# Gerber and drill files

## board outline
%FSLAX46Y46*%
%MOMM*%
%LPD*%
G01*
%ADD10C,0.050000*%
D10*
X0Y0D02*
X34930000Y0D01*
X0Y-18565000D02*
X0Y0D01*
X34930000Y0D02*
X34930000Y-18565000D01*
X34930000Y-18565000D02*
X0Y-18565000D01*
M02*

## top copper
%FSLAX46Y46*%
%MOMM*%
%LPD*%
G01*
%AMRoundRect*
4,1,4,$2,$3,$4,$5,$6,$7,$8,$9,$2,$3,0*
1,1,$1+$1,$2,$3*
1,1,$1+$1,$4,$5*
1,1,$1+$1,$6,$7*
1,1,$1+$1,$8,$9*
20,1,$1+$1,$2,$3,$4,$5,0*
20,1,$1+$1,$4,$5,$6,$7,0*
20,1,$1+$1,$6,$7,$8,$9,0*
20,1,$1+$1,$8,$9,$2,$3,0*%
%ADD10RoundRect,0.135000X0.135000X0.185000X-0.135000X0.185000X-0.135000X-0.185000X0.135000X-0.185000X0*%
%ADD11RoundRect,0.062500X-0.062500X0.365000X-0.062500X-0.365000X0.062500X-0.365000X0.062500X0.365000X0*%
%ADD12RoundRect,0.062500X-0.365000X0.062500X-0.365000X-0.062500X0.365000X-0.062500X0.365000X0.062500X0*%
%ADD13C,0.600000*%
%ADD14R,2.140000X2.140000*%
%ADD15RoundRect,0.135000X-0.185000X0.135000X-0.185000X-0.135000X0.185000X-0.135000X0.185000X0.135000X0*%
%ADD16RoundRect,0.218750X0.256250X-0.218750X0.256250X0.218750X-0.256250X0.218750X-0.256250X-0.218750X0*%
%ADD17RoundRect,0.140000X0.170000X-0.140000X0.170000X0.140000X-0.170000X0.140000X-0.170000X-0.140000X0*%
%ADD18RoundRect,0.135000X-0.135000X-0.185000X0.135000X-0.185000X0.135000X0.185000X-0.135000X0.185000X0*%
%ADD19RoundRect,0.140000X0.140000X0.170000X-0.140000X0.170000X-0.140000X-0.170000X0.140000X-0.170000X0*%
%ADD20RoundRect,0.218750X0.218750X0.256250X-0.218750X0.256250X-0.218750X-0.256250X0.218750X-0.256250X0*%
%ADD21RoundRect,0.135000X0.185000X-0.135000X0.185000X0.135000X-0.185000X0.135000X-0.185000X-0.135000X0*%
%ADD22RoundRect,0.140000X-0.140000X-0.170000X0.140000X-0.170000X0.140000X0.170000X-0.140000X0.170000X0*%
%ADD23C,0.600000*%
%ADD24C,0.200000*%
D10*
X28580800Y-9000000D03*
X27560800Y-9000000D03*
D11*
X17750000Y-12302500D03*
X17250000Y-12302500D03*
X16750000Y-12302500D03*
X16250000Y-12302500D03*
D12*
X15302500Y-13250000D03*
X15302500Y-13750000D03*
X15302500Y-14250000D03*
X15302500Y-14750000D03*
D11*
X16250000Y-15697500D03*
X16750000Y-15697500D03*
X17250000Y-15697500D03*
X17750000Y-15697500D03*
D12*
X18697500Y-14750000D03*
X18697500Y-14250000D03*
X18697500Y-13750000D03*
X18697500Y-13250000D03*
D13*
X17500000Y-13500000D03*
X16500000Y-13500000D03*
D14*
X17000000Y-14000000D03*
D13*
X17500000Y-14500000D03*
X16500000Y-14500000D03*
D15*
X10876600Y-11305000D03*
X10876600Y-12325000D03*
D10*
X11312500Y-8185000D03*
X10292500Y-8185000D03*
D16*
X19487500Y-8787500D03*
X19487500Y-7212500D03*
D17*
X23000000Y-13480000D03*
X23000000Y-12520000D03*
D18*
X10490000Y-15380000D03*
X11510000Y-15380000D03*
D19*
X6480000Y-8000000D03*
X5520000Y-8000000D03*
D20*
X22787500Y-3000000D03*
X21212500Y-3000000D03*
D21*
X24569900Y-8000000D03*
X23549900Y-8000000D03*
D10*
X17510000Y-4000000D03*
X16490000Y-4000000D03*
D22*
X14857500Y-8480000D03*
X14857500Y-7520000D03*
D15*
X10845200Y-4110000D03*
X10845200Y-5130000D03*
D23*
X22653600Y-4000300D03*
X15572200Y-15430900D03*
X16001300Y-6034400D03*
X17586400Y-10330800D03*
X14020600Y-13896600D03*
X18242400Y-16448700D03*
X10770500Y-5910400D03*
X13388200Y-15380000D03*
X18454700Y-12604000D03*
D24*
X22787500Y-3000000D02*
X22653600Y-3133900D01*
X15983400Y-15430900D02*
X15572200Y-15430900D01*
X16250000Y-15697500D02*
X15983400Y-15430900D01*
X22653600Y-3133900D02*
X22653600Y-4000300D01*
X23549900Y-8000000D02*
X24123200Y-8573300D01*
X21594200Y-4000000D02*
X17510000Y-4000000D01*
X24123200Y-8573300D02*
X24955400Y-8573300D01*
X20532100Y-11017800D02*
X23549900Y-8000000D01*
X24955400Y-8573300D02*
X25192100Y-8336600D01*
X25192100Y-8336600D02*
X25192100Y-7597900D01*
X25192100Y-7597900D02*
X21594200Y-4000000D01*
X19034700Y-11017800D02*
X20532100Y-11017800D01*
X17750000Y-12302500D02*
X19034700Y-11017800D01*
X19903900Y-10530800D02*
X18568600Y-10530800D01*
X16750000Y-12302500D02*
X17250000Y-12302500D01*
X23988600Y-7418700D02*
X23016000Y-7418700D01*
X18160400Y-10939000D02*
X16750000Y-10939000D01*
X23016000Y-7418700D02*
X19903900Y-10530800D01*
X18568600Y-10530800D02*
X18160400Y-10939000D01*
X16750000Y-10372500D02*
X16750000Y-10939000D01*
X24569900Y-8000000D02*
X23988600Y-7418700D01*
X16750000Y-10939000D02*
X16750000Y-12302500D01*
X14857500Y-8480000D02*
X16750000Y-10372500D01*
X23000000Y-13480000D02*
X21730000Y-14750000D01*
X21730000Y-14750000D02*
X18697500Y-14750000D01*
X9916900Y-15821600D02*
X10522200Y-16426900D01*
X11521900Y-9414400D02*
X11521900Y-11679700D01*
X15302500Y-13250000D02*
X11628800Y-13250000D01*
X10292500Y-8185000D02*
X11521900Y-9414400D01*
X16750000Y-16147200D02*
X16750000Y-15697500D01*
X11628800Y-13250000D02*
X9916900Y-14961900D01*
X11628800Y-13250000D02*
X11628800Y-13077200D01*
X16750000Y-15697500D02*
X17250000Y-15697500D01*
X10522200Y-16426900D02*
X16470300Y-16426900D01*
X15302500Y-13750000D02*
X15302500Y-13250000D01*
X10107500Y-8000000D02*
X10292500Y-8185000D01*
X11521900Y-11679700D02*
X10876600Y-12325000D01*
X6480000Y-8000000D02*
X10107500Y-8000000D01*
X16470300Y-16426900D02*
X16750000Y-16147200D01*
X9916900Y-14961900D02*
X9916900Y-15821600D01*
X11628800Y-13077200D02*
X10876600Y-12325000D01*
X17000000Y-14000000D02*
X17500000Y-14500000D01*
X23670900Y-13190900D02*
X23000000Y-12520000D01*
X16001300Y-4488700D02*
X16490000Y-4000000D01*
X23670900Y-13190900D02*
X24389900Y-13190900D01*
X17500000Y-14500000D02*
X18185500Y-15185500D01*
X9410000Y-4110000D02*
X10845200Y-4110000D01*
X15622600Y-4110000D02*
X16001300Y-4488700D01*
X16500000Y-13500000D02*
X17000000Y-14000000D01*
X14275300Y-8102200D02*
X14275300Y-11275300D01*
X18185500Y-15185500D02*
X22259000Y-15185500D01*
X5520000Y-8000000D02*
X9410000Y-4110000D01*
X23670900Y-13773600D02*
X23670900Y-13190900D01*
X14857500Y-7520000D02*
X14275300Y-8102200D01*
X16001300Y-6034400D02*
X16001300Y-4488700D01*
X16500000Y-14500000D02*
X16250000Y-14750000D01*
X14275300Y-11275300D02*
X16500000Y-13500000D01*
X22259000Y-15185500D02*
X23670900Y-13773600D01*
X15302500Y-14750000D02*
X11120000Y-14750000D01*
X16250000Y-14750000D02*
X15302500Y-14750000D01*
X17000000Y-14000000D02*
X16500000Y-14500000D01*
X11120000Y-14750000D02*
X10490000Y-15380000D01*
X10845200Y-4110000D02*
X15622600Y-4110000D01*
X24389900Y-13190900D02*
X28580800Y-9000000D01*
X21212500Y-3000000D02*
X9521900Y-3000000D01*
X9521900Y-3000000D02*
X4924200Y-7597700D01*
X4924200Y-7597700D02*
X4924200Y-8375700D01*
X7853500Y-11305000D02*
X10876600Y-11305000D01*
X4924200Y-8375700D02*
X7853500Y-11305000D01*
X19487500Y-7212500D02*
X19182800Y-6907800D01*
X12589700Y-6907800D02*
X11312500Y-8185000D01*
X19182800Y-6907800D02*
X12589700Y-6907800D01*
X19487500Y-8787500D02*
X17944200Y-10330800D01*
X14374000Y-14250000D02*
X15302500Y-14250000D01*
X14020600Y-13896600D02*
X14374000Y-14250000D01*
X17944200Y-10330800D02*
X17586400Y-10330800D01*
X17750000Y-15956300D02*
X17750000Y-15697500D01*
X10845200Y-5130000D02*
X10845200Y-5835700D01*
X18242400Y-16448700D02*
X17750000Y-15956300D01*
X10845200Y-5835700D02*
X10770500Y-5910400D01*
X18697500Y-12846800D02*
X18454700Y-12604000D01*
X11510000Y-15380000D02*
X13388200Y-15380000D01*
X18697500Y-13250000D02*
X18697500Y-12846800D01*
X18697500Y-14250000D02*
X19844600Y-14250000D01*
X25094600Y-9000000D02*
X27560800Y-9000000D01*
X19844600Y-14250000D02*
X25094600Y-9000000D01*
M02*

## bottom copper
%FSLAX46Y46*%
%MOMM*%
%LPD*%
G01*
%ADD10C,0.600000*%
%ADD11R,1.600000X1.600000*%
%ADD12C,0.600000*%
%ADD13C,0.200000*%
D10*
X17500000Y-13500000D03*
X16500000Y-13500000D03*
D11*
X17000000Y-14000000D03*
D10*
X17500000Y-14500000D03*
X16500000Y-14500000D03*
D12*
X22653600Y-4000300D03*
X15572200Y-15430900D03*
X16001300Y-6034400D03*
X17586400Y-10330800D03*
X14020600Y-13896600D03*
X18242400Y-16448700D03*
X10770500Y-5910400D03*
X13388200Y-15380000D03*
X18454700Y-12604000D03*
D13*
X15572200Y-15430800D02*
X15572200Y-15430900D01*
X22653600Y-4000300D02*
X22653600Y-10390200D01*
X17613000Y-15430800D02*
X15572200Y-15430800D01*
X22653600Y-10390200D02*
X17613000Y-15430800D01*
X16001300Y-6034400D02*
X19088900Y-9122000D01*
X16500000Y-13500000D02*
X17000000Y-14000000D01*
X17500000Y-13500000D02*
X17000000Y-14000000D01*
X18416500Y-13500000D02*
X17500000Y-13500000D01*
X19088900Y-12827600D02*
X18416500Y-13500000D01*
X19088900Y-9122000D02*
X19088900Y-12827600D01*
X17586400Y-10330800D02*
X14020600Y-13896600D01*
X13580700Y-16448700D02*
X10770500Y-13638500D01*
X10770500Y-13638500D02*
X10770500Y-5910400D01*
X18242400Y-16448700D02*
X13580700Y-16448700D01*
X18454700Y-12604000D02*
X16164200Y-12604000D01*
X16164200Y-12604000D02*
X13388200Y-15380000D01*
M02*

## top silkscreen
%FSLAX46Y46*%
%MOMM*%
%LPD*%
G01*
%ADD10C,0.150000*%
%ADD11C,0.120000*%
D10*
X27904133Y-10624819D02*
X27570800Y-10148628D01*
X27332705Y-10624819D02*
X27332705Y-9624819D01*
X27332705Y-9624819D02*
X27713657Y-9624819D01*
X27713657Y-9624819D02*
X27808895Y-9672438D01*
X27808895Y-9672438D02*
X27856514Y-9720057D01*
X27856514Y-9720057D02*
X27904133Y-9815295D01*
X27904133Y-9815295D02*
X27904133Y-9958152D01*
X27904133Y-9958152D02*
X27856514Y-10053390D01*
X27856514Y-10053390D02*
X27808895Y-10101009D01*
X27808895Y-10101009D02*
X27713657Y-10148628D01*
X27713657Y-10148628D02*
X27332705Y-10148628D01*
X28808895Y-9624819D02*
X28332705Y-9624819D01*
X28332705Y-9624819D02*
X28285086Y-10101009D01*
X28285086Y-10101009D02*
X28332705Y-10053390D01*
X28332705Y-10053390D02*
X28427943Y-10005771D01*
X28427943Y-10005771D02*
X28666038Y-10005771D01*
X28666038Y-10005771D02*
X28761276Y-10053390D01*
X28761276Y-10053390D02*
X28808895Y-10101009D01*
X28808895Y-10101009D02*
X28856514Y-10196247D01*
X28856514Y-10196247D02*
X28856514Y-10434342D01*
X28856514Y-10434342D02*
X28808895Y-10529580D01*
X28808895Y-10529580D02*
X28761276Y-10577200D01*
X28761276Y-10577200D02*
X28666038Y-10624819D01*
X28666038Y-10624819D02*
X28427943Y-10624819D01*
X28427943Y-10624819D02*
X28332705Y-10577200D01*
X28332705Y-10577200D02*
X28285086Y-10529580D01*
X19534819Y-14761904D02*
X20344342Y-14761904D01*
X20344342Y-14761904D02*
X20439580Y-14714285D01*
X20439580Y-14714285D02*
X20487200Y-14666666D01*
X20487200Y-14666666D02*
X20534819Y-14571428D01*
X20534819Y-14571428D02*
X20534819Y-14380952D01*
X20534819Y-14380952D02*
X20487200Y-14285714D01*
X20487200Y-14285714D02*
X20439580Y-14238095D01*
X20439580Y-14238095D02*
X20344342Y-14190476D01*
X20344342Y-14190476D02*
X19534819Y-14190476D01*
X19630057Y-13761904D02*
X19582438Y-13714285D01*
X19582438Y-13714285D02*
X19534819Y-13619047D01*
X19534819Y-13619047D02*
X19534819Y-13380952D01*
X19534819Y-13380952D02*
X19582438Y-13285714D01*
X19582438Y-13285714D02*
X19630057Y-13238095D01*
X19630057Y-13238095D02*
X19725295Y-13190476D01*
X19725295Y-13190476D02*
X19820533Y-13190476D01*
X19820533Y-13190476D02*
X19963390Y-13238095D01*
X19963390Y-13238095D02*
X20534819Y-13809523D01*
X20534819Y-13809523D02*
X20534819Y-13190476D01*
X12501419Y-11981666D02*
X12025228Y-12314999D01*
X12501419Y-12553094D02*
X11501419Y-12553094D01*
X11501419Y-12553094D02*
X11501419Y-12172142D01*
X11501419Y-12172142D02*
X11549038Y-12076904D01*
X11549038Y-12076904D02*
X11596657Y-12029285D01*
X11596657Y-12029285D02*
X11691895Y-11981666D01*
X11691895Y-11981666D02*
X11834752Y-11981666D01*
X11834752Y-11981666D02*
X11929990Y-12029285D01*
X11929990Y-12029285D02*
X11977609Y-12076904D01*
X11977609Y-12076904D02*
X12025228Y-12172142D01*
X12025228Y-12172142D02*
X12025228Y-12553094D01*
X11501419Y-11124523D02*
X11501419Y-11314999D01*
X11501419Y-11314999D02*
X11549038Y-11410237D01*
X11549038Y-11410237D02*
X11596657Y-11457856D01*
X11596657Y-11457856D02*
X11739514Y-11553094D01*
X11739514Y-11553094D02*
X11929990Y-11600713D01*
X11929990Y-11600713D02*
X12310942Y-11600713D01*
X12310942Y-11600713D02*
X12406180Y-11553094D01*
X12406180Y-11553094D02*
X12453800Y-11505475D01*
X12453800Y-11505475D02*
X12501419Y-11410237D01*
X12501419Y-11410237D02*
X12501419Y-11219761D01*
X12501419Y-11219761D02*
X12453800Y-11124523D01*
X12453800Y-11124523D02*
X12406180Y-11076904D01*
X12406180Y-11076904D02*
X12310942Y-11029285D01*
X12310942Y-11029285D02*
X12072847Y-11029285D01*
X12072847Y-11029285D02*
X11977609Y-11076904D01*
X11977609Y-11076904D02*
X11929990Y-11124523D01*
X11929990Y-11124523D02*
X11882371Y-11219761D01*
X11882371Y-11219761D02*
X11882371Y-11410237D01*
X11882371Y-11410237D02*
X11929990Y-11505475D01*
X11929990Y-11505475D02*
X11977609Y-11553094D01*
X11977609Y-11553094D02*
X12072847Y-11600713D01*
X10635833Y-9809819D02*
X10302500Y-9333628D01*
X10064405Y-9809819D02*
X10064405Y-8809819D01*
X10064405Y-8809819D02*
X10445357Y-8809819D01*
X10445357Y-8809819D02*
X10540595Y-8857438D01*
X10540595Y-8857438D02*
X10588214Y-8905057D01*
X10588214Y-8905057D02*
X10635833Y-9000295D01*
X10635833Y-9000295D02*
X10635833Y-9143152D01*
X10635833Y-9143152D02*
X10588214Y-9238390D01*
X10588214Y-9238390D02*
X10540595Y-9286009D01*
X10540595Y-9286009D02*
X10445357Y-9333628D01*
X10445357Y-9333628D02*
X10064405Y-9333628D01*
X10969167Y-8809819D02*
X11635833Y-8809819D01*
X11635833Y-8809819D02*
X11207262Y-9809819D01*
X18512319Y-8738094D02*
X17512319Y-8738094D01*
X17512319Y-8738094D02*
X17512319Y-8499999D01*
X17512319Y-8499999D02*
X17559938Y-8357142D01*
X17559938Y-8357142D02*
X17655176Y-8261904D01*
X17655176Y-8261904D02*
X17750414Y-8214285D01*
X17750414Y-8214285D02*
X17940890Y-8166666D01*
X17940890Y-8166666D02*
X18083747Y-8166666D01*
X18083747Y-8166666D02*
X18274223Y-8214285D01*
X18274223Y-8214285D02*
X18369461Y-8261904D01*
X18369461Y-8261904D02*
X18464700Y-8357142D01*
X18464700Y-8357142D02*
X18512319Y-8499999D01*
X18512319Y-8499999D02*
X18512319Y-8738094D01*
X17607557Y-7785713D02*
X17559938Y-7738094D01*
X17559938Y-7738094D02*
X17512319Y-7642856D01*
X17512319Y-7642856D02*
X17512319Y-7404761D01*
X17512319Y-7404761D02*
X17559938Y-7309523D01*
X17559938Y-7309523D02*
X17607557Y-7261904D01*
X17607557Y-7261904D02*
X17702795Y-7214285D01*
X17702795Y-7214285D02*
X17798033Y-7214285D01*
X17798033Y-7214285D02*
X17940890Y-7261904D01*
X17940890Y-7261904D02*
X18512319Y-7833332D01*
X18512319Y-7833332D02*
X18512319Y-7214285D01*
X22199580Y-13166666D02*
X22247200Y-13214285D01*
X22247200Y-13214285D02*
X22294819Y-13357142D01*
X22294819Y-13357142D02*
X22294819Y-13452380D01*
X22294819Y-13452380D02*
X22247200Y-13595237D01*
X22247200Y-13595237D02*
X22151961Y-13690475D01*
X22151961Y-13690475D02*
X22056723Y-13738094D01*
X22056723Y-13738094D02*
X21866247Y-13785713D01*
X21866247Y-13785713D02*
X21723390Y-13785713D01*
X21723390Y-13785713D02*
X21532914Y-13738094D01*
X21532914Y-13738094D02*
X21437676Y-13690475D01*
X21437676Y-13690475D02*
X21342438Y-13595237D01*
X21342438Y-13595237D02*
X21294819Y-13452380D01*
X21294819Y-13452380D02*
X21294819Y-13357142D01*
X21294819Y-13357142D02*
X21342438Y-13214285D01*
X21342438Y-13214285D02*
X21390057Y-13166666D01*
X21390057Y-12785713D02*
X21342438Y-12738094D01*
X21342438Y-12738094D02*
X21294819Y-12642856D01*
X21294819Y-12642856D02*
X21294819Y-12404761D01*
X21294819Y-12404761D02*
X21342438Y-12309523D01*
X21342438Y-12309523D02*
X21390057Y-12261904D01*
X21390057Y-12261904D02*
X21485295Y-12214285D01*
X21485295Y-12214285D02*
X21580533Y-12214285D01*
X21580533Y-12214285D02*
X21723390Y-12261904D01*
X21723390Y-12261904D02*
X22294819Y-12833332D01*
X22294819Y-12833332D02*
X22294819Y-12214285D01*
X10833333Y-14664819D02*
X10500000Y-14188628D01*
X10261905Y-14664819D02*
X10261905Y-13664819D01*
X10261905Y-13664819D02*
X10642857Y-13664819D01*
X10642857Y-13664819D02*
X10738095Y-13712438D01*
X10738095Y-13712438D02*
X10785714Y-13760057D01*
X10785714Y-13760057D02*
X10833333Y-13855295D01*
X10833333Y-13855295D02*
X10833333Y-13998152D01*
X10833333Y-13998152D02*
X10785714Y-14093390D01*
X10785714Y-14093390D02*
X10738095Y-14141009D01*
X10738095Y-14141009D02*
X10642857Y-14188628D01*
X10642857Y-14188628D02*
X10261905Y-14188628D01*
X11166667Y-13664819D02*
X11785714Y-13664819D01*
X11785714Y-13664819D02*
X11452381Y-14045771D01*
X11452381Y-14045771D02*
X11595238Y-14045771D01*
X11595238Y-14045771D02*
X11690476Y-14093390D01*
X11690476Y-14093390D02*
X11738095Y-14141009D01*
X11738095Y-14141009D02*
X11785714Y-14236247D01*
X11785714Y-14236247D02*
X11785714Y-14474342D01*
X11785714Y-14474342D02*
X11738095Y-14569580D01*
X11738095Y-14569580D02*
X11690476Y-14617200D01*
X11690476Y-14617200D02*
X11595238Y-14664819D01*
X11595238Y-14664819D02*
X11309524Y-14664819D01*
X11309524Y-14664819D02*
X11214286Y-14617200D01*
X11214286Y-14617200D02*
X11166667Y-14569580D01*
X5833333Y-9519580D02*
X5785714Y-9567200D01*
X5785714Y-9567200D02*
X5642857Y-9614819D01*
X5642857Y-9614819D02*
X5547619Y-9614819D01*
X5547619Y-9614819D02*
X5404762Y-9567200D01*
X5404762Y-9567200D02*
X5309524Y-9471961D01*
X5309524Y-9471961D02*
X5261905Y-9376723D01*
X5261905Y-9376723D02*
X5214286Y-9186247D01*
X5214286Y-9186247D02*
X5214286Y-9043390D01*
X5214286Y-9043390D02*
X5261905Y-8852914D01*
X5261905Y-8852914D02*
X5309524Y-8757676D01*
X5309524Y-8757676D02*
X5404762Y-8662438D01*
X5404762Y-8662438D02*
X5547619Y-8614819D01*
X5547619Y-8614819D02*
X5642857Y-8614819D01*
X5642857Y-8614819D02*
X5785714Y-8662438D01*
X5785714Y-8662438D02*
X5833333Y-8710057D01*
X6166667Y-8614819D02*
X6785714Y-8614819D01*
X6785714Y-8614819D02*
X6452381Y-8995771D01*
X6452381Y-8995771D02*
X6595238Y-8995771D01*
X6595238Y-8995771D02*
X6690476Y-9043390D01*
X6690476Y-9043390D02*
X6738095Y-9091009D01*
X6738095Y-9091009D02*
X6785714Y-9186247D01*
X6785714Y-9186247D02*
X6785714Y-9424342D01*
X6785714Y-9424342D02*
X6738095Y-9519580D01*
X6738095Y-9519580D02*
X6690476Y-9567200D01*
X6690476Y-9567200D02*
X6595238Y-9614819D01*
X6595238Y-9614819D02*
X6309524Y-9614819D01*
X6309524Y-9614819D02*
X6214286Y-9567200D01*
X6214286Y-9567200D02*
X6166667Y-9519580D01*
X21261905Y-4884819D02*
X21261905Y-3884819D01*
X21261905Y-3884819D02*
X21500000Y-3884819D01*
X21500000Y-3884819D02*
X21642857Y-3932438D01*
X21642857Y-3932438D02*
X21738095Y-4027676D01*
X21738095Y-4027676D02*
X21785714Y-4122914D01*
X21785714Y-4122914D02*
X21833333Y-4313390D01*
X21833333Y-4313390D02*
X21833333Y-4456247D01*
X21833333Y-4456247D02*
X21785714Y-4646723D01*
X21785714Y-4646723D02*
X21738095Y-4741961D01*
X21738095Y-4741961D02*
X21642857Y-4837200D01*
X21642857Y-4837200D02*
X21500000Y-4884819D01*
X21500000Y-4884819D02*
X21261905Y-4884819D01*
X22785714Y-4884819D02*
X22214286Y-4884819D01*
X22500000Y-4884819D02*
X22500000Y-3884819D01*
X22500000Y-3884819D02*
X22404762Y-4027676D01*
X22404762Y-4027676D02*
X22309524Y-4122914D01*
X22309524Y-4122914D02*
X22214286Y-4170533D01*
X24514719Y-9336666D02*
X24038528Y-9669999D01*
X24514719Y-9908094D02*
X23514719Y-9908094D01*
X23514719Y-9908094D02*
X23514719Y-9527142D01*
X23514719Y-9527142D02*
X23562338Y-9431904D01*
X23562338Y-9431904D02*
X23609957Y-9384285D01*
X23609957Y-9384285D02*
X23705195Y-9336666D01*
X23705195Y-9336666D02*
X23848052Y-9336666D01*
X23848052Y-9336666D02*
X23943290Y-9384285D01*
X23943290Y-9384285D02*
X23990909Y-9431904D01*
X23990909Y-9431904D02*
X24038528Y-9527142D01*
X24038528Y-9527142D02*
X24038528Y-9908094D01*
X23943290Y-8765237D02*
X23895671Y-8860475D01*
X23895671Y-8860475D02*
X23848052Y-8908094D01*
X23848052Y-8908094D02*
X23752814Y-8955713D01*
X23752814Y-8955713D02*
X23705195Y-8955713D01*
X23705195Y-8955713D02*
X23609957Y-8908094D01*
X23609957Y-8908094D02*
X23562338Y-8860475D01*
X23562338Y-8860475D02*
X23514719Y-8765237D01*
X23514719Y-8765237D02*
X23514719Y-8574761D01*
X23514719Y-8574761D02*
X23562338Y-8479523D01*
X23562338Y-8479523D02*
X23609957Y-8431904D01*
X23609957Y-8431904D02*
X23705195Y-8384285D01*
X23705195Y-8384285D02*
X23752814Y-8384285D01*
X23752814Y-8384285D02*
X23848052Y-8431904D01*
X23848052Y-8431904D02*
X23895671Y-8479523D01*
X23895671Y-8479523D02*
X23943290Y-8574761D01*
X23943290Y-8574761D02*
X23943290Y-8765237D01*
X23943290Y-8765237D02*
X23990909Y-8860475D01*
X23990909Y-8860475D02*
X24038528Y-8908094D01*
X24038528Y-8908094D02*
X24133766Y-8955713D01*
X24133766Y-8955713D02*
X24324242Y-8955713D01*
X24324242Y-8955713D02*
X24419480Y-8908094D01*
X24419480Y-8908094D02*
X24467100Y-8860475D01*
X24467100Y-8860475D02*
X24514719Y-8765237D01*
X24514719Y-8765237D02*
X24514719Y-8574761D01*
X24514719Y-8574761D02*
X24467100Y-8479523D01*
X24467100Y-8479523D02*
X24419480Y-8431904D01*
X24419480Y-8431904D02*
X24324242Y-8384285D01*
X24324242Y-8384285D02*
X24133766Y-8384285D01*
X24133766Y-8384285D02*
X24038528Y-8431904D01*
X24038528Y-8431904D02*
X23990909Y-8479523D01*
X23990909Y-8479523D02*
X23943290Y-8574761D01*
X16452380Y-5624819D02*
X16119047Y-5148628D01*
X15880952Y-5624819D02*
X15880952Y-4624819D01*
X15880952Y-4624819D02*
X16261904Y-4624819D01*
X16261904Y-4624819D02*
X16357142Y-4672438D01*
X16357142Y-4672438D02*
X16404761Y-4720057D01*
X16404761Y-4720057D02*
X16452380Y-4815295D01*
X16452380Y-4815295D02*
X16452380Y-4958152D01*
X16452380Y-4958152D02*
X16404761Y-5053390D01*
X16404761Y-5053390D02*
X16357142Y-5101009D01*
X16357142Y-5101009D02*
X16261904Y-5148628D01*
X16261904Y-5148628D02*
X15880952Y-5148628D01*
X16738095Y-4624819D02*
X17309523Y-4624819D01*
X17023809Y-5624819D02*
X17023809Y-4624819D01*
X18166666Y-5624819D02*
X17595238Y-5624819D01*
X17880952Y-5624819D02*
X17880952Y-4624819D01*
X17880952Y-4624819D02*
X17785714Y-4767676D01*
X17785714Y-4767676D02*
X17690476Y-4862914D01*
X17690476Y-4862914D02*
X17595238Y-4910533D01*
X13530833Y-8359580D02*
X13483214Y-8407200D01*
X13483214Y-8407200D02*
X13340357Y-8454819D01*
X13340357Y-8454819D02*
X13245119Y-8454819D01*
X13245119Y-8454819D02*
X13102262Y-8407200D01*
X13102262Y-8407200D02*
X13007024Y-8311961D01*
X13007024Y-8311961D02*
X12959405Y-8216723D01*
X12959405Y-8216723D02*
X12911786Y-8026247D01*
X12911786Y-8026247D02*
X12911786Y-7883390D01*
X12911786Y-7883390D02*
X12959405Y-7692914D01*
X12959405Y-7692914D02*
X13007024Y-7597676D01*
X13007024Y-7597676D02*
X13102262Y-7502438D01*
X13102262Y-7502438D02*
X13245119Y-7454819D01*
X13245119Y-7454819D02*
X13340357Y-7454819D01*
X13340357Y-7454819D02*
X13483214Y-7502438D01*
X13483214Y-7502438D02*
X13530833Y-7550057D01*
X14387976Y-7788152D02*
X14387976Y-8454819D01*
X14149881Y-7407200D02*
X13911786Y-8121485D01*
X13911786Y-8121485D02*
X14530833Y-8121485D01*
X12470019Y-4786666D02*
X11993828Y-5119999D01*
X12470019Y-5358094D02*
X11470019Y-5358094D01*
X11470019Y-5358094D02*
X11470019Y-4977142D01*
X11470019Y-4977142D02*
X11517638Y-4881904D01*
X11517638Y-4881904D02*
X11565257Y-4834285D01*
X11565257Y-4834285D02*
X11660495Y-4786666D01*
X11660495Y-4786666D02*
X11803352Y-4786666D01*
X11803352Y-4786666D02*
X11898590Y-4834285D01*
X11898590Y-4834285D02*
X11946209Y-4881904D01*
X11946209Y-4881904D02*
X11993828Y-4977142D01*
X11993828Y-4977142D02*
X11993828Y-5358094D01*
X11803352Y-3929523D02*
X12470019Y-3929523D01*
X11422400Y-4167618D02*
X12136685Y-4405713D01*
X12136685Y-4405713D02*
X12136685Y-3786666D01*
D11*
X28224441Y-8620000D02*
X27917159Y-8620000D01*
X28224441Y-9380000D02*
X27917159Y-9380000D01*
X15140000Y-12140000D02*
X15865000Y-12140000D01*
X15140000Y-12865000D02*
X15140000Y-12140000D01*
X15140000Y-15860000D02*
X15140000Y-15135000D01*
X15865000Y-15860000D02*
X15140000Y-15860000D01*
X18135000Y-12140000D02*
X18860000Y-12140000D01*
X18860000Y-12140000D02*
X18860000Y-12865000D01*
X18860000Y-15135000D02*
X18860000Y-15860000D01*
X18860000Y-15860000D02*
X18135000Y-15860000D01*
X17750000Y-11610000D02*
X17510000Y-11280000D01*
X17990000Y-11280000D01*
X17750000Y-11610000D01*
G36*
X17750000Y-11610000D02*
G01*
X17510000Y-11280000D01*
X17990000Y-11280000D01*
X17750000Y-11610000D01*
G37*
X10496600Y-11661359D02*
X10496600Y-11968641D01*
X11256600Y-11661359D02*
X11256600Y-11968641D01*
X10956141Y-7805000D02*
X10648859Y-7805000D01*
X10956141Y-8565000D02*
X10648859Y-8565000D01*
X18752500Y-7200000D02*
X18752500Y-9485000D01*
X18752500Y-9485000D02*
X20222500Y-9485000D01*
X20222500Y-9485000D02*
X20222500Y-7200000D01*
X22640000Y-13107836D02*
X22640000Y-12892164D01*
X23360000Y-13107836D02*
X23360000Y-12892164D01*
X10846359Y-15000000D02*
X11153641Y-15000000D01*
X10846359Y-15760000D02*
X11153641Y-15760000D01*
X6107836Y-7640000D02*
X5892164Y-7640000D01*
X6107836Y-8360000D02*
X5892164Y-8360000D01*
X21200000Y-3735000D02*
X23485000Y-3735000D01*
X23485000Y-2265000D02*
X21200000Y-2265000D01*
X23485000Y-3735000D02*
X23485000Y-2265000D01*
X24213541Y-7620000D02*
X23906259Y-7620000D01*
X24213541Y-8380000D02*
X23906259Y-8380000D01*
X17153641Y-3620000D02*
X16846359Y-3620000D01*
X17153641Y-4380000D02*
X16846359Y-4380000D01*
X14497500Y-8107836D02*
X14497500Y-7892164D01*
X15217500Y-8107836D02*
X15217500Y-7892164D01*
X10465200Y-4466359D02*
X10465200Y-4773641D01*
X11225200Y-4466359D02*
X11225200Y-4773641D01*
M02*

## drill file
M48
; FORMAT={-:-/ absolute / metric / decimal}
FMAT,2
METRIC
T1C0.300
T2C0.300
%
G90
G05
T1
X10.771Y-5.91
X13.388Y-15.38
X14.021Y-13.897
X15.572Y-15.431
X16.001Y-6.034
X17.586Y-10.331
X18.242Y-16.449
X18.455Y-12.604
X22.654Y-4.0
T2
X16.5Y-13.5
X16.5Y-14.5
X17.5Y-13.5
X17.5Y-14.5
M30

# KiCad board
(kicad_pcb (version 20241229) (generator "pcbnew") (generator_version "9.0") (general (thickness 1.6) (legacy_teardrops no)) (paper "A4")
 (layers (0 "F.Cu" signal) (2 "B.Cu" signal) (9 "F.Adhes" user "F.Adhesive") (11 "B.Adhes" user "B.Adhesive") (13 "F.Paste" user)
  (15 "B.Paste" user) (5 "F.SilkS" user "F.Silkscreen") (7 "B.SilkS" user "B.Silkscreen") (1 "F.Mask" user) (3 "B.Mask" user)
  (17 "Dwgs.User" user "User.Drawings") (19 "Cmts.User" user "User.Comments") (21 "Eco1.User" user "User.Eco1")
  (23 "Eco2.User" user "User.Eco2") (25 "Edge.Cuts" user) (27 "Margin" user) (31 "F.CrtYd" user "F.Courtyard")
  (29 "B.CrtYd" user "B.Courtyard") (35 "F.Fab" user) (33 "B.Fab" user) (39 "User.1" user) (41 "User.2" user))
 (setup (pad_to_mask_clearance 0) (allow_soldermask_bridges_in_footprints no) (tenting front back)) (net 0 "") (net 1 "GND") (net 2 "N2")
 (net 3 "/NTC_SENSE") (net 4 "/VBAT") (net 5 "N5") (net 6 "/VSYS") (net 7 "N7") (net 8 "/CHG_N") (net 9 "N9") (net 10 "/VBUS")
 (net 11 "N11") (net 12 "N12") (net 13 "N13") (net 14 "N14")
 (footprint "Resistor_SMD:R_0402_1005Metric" (layer "F.Cu") (at 28.0708 9 180)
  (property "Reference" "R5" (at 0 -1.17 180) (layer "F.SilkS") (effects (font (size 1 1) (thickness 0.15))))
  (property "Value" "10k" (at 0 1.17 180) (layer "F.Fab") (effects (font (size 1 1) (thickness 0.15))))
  (fp_line (start -0.153641 0.38) (end 0.153641 0.38) (stroke (width 0.12) (type solid)) (layer "F.SilkS"))
  (fp_line (start -0.153641 -0.38) (end 0.153641 -0.38) (stroke (width 0.12) (type solid)) (layer "F.SilkS"))
  (pad "1" smd roundrect (at -0.51 0 180) (size 0.54 0.64) (layers "F.Cu" "F.Mask" "F.Paste") (roundrect_rratio 0.25) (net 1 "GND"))
  (pad "2" smd roundrect (at 0.51 0 180) (size 0.54 0.64) (layers "F.Cu" "F.Mask" "F.Paste") (roundrect_rratio 0.25) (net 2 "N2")))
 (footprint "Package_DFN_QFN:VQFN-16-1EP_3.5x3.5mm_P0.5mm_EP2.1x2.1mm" (layer "F.Cu") (at 17 14 -90)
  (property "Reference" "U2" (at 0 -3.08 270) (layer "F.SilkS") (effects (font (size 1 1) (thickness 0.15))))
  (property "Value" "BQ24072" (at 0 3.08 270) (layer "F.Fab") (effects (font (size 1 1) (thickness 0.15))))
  (fp_line (start -1.86 1.86) (end -1.86 1.135) (stroke (width 0.12) (type solid)) (layer "F.SilkS"))
  (fp_line (start -1.135 1.86) (end -1.86 1.86) (stroke (width 0.12) (type solid)) (layer "F.SilkS"))
  (fp_line (start 1.86 1.86) (end 1.135 1.86) (stroke (width 0.12) (type solid)) (layer "F.SilkS"))
  (fp_line (start 1.86 1.135) (end 1.86 1.86) (stroke (width 0.12) (type solid)) (layer "F.SilkS"))
  (fp_line (start -1.86 -1.135) (end -1.86 -1.86) (stroke (width 0.12) (type solid)) (layer "F.SilkS"))
  (fp_line (start -1.86 -1.86) (end -1.135 -1.86) (stroke (width 0.12) (type solid)) (layer "F.SilkS"))
  (fp_line (start 1.135 -1.86) (end 1.86 -1.86) (stroke (width 0.12) (type solid)) (layer "F.SilkS"))
  (fp_line (start 1.86 -1.86) (end 1.86 -1.135) (stroke (width 0.12) (type solid)) (layer "F.SilkS"))
  (fp_poly (pts (xy -2.39 -0.75) (xy -2.72 -0.51) (xy -2.72 -0.99)) (stroke (width 0.12) (type solid)) (fill yes) (layer "F.SilkS"))
  (pad "" smd roundrect (at -0.535 -0.535 270) (size 0.85 0.85) (layers "F.Paste") (roundrect_rratio 0.25))
  (pad "" smd roundrect (at -0.535 0.535 270) (size 0.85 0.85) (layers "F.Paste") (roundrect_rratio 0.25))
  (pad "" smd roundrect (at 0.535 -0.535 270) (size 0.85 0.85) (layers "F.Paste") (roundrect_rratio 0.25))
  (pad "" smd roundrect (at 0.535 0.535 270) (size 0.85 0.85) (layers "F.Paste") (roundrect_rratio 0.25))
  (pad "1" smd roundrect (at -1.6975 -0.75 270) (size 0.855 0.25) (layers "F.Cu" "F.Mask" "F.Paste") (roundrect_rratio 0.25)
   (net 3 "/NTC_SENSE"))
  (pad "2" smd roundrect (at -1.6975 -0.25 270) (size 0.855 0.25) (layers "F.Cu" "F.Mask" "F.Paste") (roundrect_rratio 0.25) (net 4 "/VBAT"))
  (pad "3" smd roundrect (at -1.6975 0.25 270) (size 0.855 0.25) (layers "F.Cu" "F.Mask" "F.Paste") (roundrect_rratio 0.25) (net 4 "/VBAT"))
  (pad "4" smd roundrect (at -1.6975 0.75 270) (size 0.855 0.25) (layers "F.Cu" "F.Mask" "F.Paste") (roundrect_rratio 0.25) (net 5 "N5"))
  (pad "5" smd roundrect (at -0.75 1.6975 270) (size 0.25 0.855) (layers "F.Cu" "F.Mask" "F.Paste") (roundrect_rratio 0.25) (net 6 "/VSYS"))
  (pad "6" smd roundrect (at -0.25 1.6975 270) (size 0.25 0.855) (layers "F.Cu" "F.Mask" "F.Paste") (roundrect_rratio 0.25) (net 6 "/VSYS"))
  (pad "7" smd roundrect (at 0.25 1.6975 270) (size 0.25 0.855) (layers "F.Cu" "F.Mask" "F.Paste") (roundrect_rratio 0.25) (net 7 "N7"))
  (pad "8" smd roundrect (at 0.75 1.6975 270) (size 0.25 0.855) (layers "F.Cu" "F.Mask" "F.Paste") (roundrect_rratio 0.25) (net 1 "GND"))
  (pad "9" smd roundrect (at 1.6975 0.75 270) (size 0.855 0.25) (layers "F.Cu" "F.Mask" "F.Paste") (roundrect_rratio 0.25) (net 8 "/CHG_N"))
  (pad "10" smd roundrect (at 1.6975 0.25 270) (size 0.855 0.25) (layers "F.Cu" "F.Mask" "F.Paste") (roundrect_rratio 0.25) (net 6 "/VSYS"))
  (pad "11" smd roundrect (at 1.6975 -0.25 270) (size 0.855 0.25) (layers "F.Cu" "F.Mask" "F.Paste") (roundrect_rratio 0.25) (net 6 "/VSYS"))
  (pad "12" smd roundrect (at 1.6975 -0.75 270) (size 0.855 0.25) (layers "F.Cu" "F.Mask" "F.Paste") (roundrect_rratio 0.25) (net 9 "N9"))
  (pad "13" smd roundrect (at 0.75 -1.6975 270) (size 0.25 0.855) (layers "F.Cu" "F.Mask" "F.Paste") (roundrect_rratio 0.25)
   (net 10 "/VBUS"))
  (pad "14" smd roundrect (at 0.25 -1.6975 270) (size 0.25 0.855) (layers "F.Cu" "F.Mask" "F.Paste") (roundrect_rratio 0.25) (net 2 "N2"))
  (pad "15" smd roundrect (at -0.25 -1.6975 270) (size 0.25 0.855) (layers "F.Cu" "F.Mask" "F.Paste") (roundrect_rratio 0.25) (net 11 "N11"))
  (pad "16" smd roundrect (at -0.75 -1.6975 270) (size 0.25 0.855) (layers "F.Cu" "F.Mask" "F.Paste") (roundrect_rratio 0.25) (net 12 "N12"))
  (pad "17" thru_hole circle (at -0.5 -0.5 270) (size 0.6 0.6) (drill 0.3) (layers "*.Cu") (remove_unused_layers no) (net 1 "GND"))
  (pad "17" thru_hole circle (at -0.5 0.5 270) (size 0.6 0.6) (drill 0.3) (layers "*.Cu") (remove_unused_layers no) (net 1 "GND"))
  (pad "17" smd rect (at 0 0 270) (size 1.6 1.6) (layers "B.Cu") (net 1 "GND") (zone_connect 2))
  (pad "17" smd rect (at 0 0 270) (size 2.14 2.14) (layers "F.Cu" "F.Mask") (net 1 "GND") (zone_connect 2))
  (pad "17" thru_hole circle (at 0.5 -0.5 270) (size 0.6 0.6) (drill 0.3) (layers "*.Cu") (remove_unused_layers no) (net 1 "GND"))
  (pad "17" thru_hole circle (at 0.5 0.5 270) (size 0.6 0.6) (drill 0.3) (layers "*.Cu") (remove_unused_layers no) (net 1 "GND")))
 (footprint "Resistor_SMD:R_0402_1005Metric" (layer "F.Cu") (at 10.8766 11.815 -90)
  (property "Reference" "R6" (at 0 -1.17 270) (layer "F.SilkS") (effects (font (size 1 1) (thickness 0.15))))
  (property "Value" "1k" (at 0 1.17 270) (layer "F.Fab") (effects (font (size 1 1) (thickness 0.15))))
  (fp_line (start -0.153641 0.38) (end 0.153641 0.38) (stroke (width 0.12) (type solid)) (layer "F.SilkS"))
  (fp_line (start -0.153641 -0.38) (end 0.153641 -0.38) (stroke (width 0.12) (type solid)) (layer "F.SilkS"))
  (pad "1" smd roundrect (at -0.51 0 270) (size 0.54 0.64) (layers "F.Cu" "F.Mask" "F.Paste") (roundrect_rratio 0.25) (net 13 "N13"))
  (pad "2" smd roundrect (at 0.51 0 270) (size 0.54 0.64) (layers "F.Cu" "F.Mask" "F.Paste") (roundrect_rratio 0.25) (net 6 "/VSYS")))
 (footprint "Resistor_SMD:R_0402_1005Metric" (layer "F.Cu") (at 10.8025 8.185 180)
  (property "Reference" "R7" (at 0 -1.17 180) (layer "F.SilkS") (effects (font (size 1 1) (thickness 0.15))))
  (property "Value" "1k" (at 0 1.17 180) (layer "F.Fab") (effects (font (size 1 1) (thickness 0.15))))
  (fp_line (start -0.153641 0.38) (end 0.153641 0.38) (stroke (width 0.12) (type solid)) (layer "F.SilkS"))
  (fp_line (start -0.153641 -0.38) (end 0.153641 -0.38) (stroke (width 0.12) (type solid)) (layer "F.SilkS"))
  (pad "1" smd roundrect (at -0.51 0 180) (size 0.54 0.64) (layers "F.Cu" "F.Mask" "F.Paste") (roundrect_rratio 0.25) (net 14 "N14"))
  (pad "2" smd roundrect (at 0.51 0 180) (size 0.54 0.64) (layers "F.Cu" "F.Mask" "F.Paste") (roundrect_rratio 0.25) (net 6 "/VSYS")))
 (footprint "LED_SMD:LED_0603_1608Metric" (layer "F.Cu") (at 19.4875 8 90)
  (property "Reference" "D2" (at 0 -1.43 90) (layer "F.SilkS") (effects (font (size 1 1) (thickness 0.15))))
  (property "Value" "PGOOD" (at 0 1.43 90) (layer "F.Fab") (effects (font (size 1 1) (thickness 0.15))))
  (fp_line (start 0.8 -0.735) (end -1.485 -0.735) (stroke (width 0.12) (type solid)) (layer "F.SilkS"))
  (fp_line (start -1.485 -0.735) (end -1.485 0.735) (stroke (width 0.12) (type solid)) (layer "F.SilkS"))
  (fp_line (start -1.485 0.735) (end 0.8 0.735) (stroke (width 0.12) (type solid)) (layer "F.SilkS"))
  (pad "1" smd roundrect (at -0.7875 0 90) (size 0.875 0.95) (layers "F.Cu" "F.Mask" "F.Paste") (roundrect_rratio 0.25) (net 7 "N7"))
  (pad "2" smd roundrect (at 0.7875 0 90) (size 0.875 0.95) (layers "F.Cu" "F.Mask" "F.Paste") (roundrect_rratio 0.25) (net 14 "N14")))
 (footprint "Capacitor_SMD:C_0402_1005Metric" (layer "F.Cu") (at 23 13 90)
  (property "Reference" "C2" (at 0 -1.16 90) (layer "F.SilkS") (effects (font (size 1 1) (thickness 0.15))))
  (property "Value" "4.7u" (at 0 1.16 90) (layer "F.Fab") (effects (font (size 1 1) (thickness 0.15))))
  (fp_line (start -0.107836 -0.36) (end 0.107836 -0.36) (stroke (width 0.12) (type solid)) (layer "F.SilkS"))
  (fp_line (start -0.107836 0.36) (end 0.107836 0.36) (stroke (width 0.12) (type solid)) (layer "F.SilkS"))
  (pad "1" smd roundrect (at -0.48 0 90) (size 0.56 0.62) (layers "F.Cu" "F.Mask" "F.Paste") (roundrect_rratio 0.25) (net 10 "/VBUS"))
  (pad "2" smd roundrect (at 0.48 0 90) (size 0.56 0.62) (layers "F.Cu" "F.Mask" "F.Paste") (roundrect_rratio 0.25) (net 1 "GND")))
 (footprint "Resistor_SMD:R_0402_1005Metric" (layer "F.Cu") (at 11 15.38)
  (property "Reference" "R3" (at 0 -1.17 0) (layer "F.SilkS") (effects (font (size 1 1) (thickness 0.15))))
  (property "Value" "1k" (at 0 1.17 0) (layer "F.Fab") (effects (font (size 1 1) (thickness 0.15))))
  (fp_line (start -0.153641 -0.38) (end 0.153641 -0.38) (stroke (width 0.12) (type solid)) (layer "F.SilkS"))
  (fp_line (start -0.153641 0.38) (end 0.153641 0.38) (stroke (width 0.12) (type solid)) (layer "F.SilkS"))
  (pad "1" smd roundrect (at -0.51 0) (size 0.54 0.64) (layers "F.Cu" "F.Mask" "F.Paste") (roundrect_rratio 0.25) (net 1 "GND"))
  (pad "2" smd roundrect (at 0.51 0) (size 0.54 0.64) (layers "F.Cu" "F.Mask" "F.Paste") (roundrect_rratio 0.25) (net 12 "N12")))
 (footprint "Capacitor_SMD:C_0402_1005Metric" (layer "F.Cu") (at 6 8 180)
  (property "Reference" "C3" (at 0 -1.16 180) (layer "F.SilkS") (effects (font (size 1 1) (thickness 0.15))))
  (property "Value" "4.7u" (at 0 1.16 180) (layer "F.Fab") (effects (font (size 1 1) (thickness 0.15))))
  (fp_line (start -0.107836 0.36) (end 0.107836 0.36) (stroke (width 0.12) (type solid)) (layer "F.SilkS"))
  (fp_line (start -0.107836 -0.36) (end 0.107836 -0.36) (stroke (width 0.12) (type solid)) (layer "F.SilkS"))
  (pad "1" smd roundrect (at -0.48 0 180) (size 0.56 0.62) (layers "F.Cu" "F.Mask" "F.Paste") (roundrect_rratio 0.25) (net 6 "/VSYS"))
  (pad "2" smd roundrect (at 0.48 0 180) (size 0.56 0.62) (layers "F.Cu" "F.Mask" "F.Paste") (roundrect_rratio 0.25) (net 1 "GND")))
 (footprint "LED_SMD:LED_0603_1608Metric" (layer "F.Cu") (at 22 3 180)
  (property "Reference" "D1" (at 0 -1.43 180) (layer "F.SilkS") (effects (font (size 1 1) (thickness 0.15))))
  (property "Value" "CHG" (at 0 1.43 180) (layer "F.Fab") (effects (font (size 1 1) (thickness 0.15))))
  (fp_line (start 0.8 -0.735) (end -1.485 -0.735) (stroke (width 0.12) (type solid)) (layer "F.SilkS"))
  (fp_line (start -1.485 0.735) (end 0.8 0.735) (stroke (width 0.12) (type solid)) (layer "F.SilkS"))
  (fp_line (start -1.485 -0.735) (end -1.485 0.735) (stroke (width 0.12) (type solid)) (layer "F.SilkS"))
  (pad "1" smd roundrect (at -0.7875 0 180) (size 0.875 0.95) (layers "F.Cu" "F.Mask" "F.Paste") (roundrect_rratio 0.25) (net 8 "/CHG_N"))
  (pad "2" smd roundrect (at 0.7875 0 180) (size 0.875 0.95) (layers "F.Cu" "F.Mask" "F.Paste") (roundrect_rratio 0.25) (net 13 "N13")))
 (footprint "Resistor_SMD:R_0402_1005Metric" (layer "F.Cu") (at 24.0599 8 180)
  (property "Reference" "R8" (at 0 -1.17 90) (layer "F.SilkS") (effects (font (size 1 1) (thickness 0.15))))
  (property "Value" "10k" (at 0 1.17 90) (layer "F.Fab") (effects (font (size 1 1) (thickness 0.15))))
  (fp_line (start -0.153641 0.38) (end 0.153641 0.38) (stroke (width 0.12) (type solid)) (layer "F.SilkS"))
  (fp_line (start -0.153641 -0.38) (end 0.153641 -0.38) (stroke (width 0.12) (type solid)) (layer "F.SilkS"))
  (pad "1" smd roundrect (at -0.51 0 90) (size 0.54 0.64) (layers "F.Cu" "F.Mask" "F.Paste") (roundrect_rratio 0.25) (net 4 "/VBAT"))
  (pad "2" smd roundrect (at 0.51 0 90) (size 0.54 0.64) (layers "F.Cu" "F.Mask" "F.Paste") (roundrect_rratio 0.25) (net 3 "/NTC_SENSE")))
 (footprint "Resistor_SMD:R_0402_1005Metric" (layer "F.Cu") (at 17 4 180)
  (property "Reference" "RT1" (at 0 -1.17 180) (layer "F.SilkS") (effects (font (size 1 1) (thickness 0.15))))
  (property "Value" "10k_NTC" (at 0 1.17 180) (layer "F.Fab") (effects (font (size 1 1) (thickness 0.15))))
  (fp_line (start -0.153641 0.38) (end 0.153641 0.38) (stroke (width 0.12) (type solid)) (layer "F.SilkS"))
  (fp_line (start -0.153641 -0.38) (end 0.153641 -0.38) (stroke (width 0.12) (type solid)) (layer "F.SilkS"))
  (pad "1" smd roundrect (at -0.51 0 180) (size 0.54 0.64) (layers "F.Cu" "F.Mask" "F.Paste") (roundrect_rratio 0.25) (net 3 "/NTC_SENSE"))
  (pad "2" smd roundrect (at 0.51 0 180) (size 0.54 0.64) (layers "F.Cu" "F.Mask" "F.Paste") (roundrect_rratio 0.25) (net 1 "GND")))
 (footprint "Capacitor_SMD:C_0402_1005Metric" (layer "F.Cu") (at 14.8575 8 90)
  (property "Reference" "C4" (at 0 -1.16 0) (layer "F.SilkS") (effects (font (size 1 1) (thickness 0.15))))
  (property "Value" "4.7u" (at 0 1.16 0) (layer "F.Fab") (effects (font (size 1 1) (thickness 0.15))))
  (fp_line (start -0.107836 -0.36) (end 0.107836 -0.36) (stroke (width 0.12) (type solid)) (layer "F.SilkS"))
  (fp_line (start -0.107836 0.36) (end 0.107836 0.36) (stroke (width 0.12) (type solid)) (layer "F.SilkS"))
  (pad "1" smd roundrect (at -0.48 0) (size 0.56 0.62) (layers "F.Cu" "F.Mask" "F.Paste") (roundrect_rratio 0.25) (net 4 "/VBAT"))
  (pad "2" smd roundrect (at 0.48 0) (size 0.56 0.62) (layers "F.Cu" "F.Mask" "F.Paste") (roundrect_rratio 0.25) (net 1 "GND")))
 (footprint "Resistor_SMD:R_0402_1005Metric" (layer "F.Cu") (at 10.8452 4.62 -90)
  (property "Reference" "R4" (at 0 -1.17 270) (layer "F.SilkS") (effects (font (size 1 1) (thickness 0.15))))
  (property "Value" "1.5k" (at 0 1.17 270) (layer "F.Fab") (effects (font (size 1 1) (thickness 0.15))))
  (fp_line (start -0.153641 0.38) (end 0.153641 0.38) (stroke (width 0.12) (type solid)) (layer "F.SilkS"))
  (fp_line (start -0.153641 -0.38) (end 0.153641 -0.38) (stroke (width 0.12) (type solid)) (layer "F.SilkS"))
  (pad "1" smd roundrect (at -0.51 0 270) (size 0.54 0.64) (layers "F.Cu" "F.Mask" "F.Paste") (roundrect_rratio 0.25) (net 1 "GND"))
  (pad "2" smd roundrect (at 0.51 0 270) (size 0.54 0.64) (layers "F.Cu" "F.Mask" "F.Paste") (roundrect_rratio 0.25) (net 9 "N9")))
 (gr_line (start 0 0) (end 34.93 0) (stroke (width 0.05) (type default)) (layer "Edge.Cuts"))
 (gr_line (start 0 18.565) (end 0 0) (stroke (width 0.05) (type default)) (layer "Edge.Cuts"))
 (gr_line (start 34.93 0) (end 34.93 18.565) (stroke (width 0.05) (type default)) (layer "Edge.Cuts"))
 (gr_line (start 34.93 18.565) (end 0 18.565) (stroke (width 0.05) (type default)) (layer "Edge.Cuts"))
 (segment (start 22.7875 3) (end 22.6536 3.1339) (width 0.2) (layer "F.Cu") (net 8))
 (segment (start 15.9834 15.4309) (end 15.5722 15.4309) (width 0.2) (layer "F.Cu") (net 8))
 (segment (start 16.25 15.6975) (end 15.9834 15.4309) (width 0.2) (layer "F.Cu") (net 8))
 (segment (start 22.6536 3.1339) (end 22.6536 4.0003) (width 0.2) (layer "F.Cu") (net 8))
 (via (at 22.6536 4.0003) (size 0.6) (drill 0.3) (layers "F.Cu" "B.Cu") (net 8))
 (via (at 15.5722 15.4309) (size 0.6) (drill 0.3) (layers "F.Cu" "B.Cu") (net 8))
 (segment (start 15.5722 15.4308) (end 15.5722 15.4309) (width 0.2) (layer "B.Cu") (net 8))
 (segment (start 22.6536 4.0003) (end 22.6536 10.3902) (width 0.2) (layer "B.Cu") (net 8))
 (segment (start 17.613 15.4308) (end 15.5722 15.4308) (width 0.2) (layer "B.Cu") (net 8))
 (segment (start 22.6536 10.3902) (end 17.613 15.4308) (width 0.2) (layer "B.Cu") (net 8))
 (segment (start 23.5499 8) (end 24.1232 8.5733) (width 0.2) (layer "F.Cu") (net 3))
 (segment (start 21.5942 4) (end 17.51 4) (width 0.2) (layer "F.Cu") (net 3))
 (segment (start 24.1232 8.5733) (end 24.9554 8.5733) (width 0.2) (layer "F.Cu") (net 3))
 (segment (start 20.5321 11.0178) (end 23.5499 8) (width 0.2) (layer "F.Cu") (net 3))
 (segment (start 24.9554 8.5733) (end 25.1921 8.3366) (width 0.2) (layer "F.Cu") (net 3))
 (segment (start 25.1921 8.3366) (end 25.1921 7.5979) (width 0.2) (layer "F.Cu") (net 3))
 (segment (start 25.1921 7.5979) (end 21.5942 4) (width 0.2) (layer "F.Cu") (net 3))
 (segment (start 19.0347 11.0178) (end 20.5321 11.0178) (width 0.2) (layer "F.Cu") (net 3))
 (segment (start 17.75 12.3025) (end 19.0347 11.0178) (width 0.2) (layer "F.Cu") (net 3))
 (segment (start 19.9039 10.5308) (end 18.5686 10.5308) (width 0.2) (layer "F.Cu") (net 4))
 (segment (start 16.75 12.3025) (end 17.25 12.3025) (width 0.2) (layer "F.Cu") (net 4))
 (segment (start 23.9886 7.4187) (end 23.016 7.4187) (width 0.2) (layer "F.Cu") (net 4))
 (segment (start 18.1604 10.939) (end 16.75 10.939) (width 0.2) (layer "F.Cu") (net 4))
 (segment (start 23.016 7.4187) (end 19.9039 10.5308) (width 0.2) (layer "F.Cu") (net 4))
 (segment (start 18.5686 10.5308) (end 18.1604 10.939) (width 0.2) (layer "F.Cu") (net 4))
 (segment (start 16.75 10.3725) (end 16.75 10.939) (width 0.2) (layer "F.Cu") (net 4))
 (segment (start 24.5699 8) (end 23.9886 7.4187) (width 0.2) (layer "F.Cu") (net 4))
 (segment (start 16.75 10.939) (end 16.75 12.3025) (width 0.2) (layer "F.Cu") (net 4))
 (segment (start 14.8575 8.48) (end 16.75 10.3725) (width 0.2) (layer "F.Cu") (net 4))
 (segment (start 23 13.48) (end 21.73 14.75) (width 0.2) (layer "F.Cu") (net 10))
 (segment (start 21.73 14.75) (end 18.6975 14.75) (width 0.2) (layer "F.Cu") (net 10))
 (segment (start 9.9169 15.8216) (end 10.5222 16.4269) (width 0.2) (layer "F.Cu") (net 6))
 (segment (start 11.5219 9.4144) (end 11.5219 11.6797) (width 0.2) (layer "F.Cu") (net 6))
 (segment (start 15.3025 13.25) (end 11.6288 13.25) (width 0.2) (layer "F.Cu") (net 6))
 (segment (start 10.2925 8.185) (end 11.5219 9.4144) (width 0.2) (layer "F.Cu") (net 6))
 (segment (start 16.75 16.1472) (end 16.75 15.6975) (width 0.2) (layer "F.Cu") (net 6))
 (segment (start 11.6288 13.25) (end 9.9169 14.9619) (width 0.2) (layer "F.Cu") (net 6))
 (segment (start 11.6288 13.25) (end 11.6288 13.0772) (width 0.2) (layer "F.Cu") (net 6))
 (segment (start 16.75 15.6975) (end 17.25 15.6975) (width 0.2) (layer "F.Cu") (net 6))
 (segment (start 10.5222 16.4269) (end 16.4703 16.4269) (width 0.2) (layer "F.Cu") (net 6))
 (segment (start 15.3025 13.75) (end 15.3025 13.25) (width 0.2) (layer "F.Cu") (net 6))
 (segment (start 10.1075 8) (end 10.2925 8.185) (width 0.2) (layer "F.Cu") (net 6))
 (segment (start 11.5219 11.6797) (end 10.8766 12.325) (width 0.2) (layer "F.Cu") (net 6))
 (segment (start 6.48 8) (end 10.1075 8) (width 0.2) (layer "F.Cu") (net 6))
 (segment (start 16.4703 16.4269) (end 16.75 16.1472) (width 0.2) (layer "F.Cu") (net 6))
 (segment (start 9.9169 14.9619) (end 9.9169 15.8216) (width 0.2) (layer "F.Cu") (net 6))
 (segment (start 11.6288 13.0772) (end 10.8766 12.325) (width 0.2) (layer "F.Cu") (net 6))
 (segment (start 17 14) (end 17.5 14.5) (width 0.2) (layer "F.Cu") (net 1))
 (segment (start 23.6709 13.1909) (end 23 12.52) (width 0.2) (layer "F.Cu") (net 1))
 (segment (start 16.0013 4.4887) (end 16.49 4) (width 0.2) (layer "F.Cu") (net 1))
 (segment (start 23.6709 13.1909) (end 24.3899 13.1909) (width 0.2) (layer "F.Cu") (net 1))
 (segment (start 17.5 14.5) (end 18.1855 15.1855) (width 0.2) (layer "F.Cu") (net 1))
 (segment (start 9.41 4.11) (end 10.8452 4.11) (width 0.2) (layer "F.Cu") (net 1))
 (segment (start 15.6226 4.11) (end 16.0013 4.4887) (width 0.2) (layer "F.Cu") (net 1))
 (segment (start 16.5 13.5) (end 17 14) (width 0.2) (layer "F.Cu") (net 1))
 (segment (start 14.2753 8.1022) (end 14.2753 11.2753) (width 0.2) (layer "F.Cu") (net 1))
 (segment (start 18.1855 15.1855) (end 22.259 15.1855) (width 0.2) (layer "F.Cu") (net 1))
 (segment (start 5.52 8) (end 9.41 4.11) (width 0.2) (layer "F.Cu") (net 1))
 (segment (start 23.6709 13.7736) (end 23.6709 13.1909) (width 0.2) (layer "F.Cu") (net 1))
 (segment (start 14.8575 7.52) (end 14.2753 8.1022) (width 0.2) (layer "F.Cu") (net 1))
 (segment (start 16.0013 6.0344) (end 16.0013 4.4887) (width 0.2) (layer "F.Cu") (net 1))
 (segment (start 16.5 14.5) (end 16.25 14.75) (width 0.2) (layer "F.Cu") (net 1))
 (segment (start 14.2753 11.2753) (end 16.5 13.5) (width 0.2) (layer "F.Cu") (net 1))
 (segment (start 22.259 15.1855) (end 23.6709 13.7736) (width 0.2) (layer "F.Cu") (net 1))
 (segment (start 15.3025 14.75) (end 11.12 14.75) (width 0.2) (layer "F.Cu") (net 1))
 (segment (start 16.25 14.75) (end 15.3025 14.75) (width 0.2) (layer "F.Cu") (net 1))
 (segment (start 17 14) (end 16.5 14.5) (width 0.2) (layer "F.Cu") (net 1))
 (segment (start 11.12 14.75) (end 10.49 15.38) (width 0.2) (layer "F.Cu") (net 1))
 (segment (start 10.8452 4.11) (end 15.6226 4.11) (width 0.2) (layer "F.Cu") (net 1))
 (segment (start 24.3899 13.1909) (end 28.5808 9) (width 0.2) (layer "F.Cu") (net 1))
 (via (at 16.0013 6.0344) (size 0.6) (drill 0.3) (layers "F.Cu" "B.Cu") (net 1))
 (segment (start 16.0013 6.0344) (end 19.0889 9.122) (width 0.2) (layer "B.Cu") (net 1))
 (segment (start 16.5 13.5) (end 17 14) (width 0.2) (layer "B.Cu") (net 1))
 (segment (start 17.5 13.5) (end 17 14) (width 0.2) (layer "B.Cu") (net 1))
 (segment (start 18.4165 13.5) (end 17.5 13.5) (width 0.2) (layer "B.Cu") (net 1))
 (segment (start 19.0889 12.8276) (end 18.4165 13.5) (width 0.2) (layer "B.Cu") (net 1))
 (segment (start 19.0889 9.122) (end 19.0889 12.8276) (width 0.2) (layer "B.Cu") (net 1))
 (segment (start 21.2125 3) (end 9.5219 3) (width 0.2) (layer "F.Cu") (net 13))
 (segment (start 9.5219 3) (end 4.9242 7.5977) (width 0.2) (layer "F.Cu") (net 13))
 (segment (start 4.9242 7.5977) (end 4.9242 8.3757) (width 0.2) (layer "F.Cu") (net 13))
 (segment (start 7.8535 11.305) (end 10.8766 11.305) (width 0.2) (layer "F.Cu") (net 13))
 (segment (start 4.9242 8.3757) (end 7.8535 11.305) (width 0.2) (layer "F.Cu") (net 13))
 (segment (start 19.4875 7.2125) (end 19.1828 6.9078) (width 0.2) (layer "F.Cu") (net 14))
 (segment (start 12.5897 6.9078) (end 11.3125 8.185) (width 0.2) (layer "F.Cu") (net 14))
 (segment (start 19.1828 6.9078) (end 12.5897 6.9078) (width 0.2) (layer "F.Cu") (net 14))
 (segment (start 19.4875 8.7875) (end 17.9442 10.3308) (width 0.2) (layer "F.Cu") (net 7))
 (segment (start 14.374 14.25) (end 15.3025 14.25) (width 0.2) (layer "F.Cu") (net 7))
 (segment (start 14.0206 13.8966) (end 14.374 14.25) (width 0.2) (layer "F.Cu") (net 7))
 (segment (start 17.9442 10.3308) (end 17.5864 10.3308) (width 0.2) (layer "F.Cu") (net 7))
 (via (at 17.5864 10.3308) (size 0.6) (drill 0.3) (layers "F.Cu" "B.Cu") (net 7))
 (via (at 14.0206 13.8966) (size 0.6) (drill 0.3) (layers "F.Cu" "B.Cu") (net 7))
 (segment (start 17.5864 10.3308) (end 14.0206 13.8966) (width 0.2) (layer "B.Cu") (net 7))
 (segment (start 17.75 15.9563) (end 17.75 15.6975) (width 0.2) (layer "F.Cu") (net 9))
 (segment (start 10.8452 5.13) (end 10.8452 5.8357) (width 0.2) (layer "F.Cu") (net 9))
 (segment (start 18.2424 16.4487) (end 17.75 15.9563) (width 0.2) (layer "F.Cu") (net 9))
 (segment (start 10.8452 5.8357) (end 10.7705 5.9104) (width 0.2) (layer "F.Cu") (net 9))
 (via (at 18.2424 16.4487) (size 0.6) (drill 0.3) (layers "F.Cu" "B.Cu") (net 9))
 (via (at 10.7705 5.9104) (size 0.6) (drill 0.3) (layers "F.Cu" "B.Cu") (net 9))
 (segment (start 13.5807 16.4487) (end 10.7705 13.6385) (width 0.2) (layer "B.Cu") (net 9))
 (segment (start 10.7705 13.6385) (end 10.7705 5.9104) (width 0.2) (layer "B.Cu") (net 9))
 (segment (start 18.2424 16.4487) (end 13.5807 16.4487) (width 0.2) (layer "B.Cu") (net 9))
 (segment (start 18.6975 12.8468) (end 18.4547 12.604) (width 0.2) (layer "F.Cu") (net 12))
 (segment (start 11.51 15.38) (end 13.3882 15.38) (width 0.2) (layer "F.Cu") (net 12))
 (segment (start 18.6975 13.25) (end 18.6975 12.8468) (width 0.2) (layer "F.Cu") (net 12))
 (via (at 13.3882 15.38) (size 0.6) (drill 0.3) (layers "F.Cu" "B.Cu") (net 12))
 (via (at 18.4547 12.604) (size 0.6) (drill 0.3) (layers "F.Cu" "B.Cu") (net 12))
 (segment (start 18.4547 12.604) (end 16.1642 12.604) (width 0.2) (layer "B.Cu") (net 12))
 (segment (start 16.1642 12.604) (end 13.3882 15.38) (width 0.2) (layer "B.Cu") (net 12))
 (segment (start 18.6975 14.25) (end 19.8446 14.25) (width 0.2) (layer "F.Cu") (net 2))
 (segment (start 25.0946 9) (end 27.5608 9) (width 0.2) (layer "F.Cu") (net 2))
 (segment (start 19.8446 14.25) (end 25.0946 9) (width 0.2) (layer "F.Cu") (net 2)))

